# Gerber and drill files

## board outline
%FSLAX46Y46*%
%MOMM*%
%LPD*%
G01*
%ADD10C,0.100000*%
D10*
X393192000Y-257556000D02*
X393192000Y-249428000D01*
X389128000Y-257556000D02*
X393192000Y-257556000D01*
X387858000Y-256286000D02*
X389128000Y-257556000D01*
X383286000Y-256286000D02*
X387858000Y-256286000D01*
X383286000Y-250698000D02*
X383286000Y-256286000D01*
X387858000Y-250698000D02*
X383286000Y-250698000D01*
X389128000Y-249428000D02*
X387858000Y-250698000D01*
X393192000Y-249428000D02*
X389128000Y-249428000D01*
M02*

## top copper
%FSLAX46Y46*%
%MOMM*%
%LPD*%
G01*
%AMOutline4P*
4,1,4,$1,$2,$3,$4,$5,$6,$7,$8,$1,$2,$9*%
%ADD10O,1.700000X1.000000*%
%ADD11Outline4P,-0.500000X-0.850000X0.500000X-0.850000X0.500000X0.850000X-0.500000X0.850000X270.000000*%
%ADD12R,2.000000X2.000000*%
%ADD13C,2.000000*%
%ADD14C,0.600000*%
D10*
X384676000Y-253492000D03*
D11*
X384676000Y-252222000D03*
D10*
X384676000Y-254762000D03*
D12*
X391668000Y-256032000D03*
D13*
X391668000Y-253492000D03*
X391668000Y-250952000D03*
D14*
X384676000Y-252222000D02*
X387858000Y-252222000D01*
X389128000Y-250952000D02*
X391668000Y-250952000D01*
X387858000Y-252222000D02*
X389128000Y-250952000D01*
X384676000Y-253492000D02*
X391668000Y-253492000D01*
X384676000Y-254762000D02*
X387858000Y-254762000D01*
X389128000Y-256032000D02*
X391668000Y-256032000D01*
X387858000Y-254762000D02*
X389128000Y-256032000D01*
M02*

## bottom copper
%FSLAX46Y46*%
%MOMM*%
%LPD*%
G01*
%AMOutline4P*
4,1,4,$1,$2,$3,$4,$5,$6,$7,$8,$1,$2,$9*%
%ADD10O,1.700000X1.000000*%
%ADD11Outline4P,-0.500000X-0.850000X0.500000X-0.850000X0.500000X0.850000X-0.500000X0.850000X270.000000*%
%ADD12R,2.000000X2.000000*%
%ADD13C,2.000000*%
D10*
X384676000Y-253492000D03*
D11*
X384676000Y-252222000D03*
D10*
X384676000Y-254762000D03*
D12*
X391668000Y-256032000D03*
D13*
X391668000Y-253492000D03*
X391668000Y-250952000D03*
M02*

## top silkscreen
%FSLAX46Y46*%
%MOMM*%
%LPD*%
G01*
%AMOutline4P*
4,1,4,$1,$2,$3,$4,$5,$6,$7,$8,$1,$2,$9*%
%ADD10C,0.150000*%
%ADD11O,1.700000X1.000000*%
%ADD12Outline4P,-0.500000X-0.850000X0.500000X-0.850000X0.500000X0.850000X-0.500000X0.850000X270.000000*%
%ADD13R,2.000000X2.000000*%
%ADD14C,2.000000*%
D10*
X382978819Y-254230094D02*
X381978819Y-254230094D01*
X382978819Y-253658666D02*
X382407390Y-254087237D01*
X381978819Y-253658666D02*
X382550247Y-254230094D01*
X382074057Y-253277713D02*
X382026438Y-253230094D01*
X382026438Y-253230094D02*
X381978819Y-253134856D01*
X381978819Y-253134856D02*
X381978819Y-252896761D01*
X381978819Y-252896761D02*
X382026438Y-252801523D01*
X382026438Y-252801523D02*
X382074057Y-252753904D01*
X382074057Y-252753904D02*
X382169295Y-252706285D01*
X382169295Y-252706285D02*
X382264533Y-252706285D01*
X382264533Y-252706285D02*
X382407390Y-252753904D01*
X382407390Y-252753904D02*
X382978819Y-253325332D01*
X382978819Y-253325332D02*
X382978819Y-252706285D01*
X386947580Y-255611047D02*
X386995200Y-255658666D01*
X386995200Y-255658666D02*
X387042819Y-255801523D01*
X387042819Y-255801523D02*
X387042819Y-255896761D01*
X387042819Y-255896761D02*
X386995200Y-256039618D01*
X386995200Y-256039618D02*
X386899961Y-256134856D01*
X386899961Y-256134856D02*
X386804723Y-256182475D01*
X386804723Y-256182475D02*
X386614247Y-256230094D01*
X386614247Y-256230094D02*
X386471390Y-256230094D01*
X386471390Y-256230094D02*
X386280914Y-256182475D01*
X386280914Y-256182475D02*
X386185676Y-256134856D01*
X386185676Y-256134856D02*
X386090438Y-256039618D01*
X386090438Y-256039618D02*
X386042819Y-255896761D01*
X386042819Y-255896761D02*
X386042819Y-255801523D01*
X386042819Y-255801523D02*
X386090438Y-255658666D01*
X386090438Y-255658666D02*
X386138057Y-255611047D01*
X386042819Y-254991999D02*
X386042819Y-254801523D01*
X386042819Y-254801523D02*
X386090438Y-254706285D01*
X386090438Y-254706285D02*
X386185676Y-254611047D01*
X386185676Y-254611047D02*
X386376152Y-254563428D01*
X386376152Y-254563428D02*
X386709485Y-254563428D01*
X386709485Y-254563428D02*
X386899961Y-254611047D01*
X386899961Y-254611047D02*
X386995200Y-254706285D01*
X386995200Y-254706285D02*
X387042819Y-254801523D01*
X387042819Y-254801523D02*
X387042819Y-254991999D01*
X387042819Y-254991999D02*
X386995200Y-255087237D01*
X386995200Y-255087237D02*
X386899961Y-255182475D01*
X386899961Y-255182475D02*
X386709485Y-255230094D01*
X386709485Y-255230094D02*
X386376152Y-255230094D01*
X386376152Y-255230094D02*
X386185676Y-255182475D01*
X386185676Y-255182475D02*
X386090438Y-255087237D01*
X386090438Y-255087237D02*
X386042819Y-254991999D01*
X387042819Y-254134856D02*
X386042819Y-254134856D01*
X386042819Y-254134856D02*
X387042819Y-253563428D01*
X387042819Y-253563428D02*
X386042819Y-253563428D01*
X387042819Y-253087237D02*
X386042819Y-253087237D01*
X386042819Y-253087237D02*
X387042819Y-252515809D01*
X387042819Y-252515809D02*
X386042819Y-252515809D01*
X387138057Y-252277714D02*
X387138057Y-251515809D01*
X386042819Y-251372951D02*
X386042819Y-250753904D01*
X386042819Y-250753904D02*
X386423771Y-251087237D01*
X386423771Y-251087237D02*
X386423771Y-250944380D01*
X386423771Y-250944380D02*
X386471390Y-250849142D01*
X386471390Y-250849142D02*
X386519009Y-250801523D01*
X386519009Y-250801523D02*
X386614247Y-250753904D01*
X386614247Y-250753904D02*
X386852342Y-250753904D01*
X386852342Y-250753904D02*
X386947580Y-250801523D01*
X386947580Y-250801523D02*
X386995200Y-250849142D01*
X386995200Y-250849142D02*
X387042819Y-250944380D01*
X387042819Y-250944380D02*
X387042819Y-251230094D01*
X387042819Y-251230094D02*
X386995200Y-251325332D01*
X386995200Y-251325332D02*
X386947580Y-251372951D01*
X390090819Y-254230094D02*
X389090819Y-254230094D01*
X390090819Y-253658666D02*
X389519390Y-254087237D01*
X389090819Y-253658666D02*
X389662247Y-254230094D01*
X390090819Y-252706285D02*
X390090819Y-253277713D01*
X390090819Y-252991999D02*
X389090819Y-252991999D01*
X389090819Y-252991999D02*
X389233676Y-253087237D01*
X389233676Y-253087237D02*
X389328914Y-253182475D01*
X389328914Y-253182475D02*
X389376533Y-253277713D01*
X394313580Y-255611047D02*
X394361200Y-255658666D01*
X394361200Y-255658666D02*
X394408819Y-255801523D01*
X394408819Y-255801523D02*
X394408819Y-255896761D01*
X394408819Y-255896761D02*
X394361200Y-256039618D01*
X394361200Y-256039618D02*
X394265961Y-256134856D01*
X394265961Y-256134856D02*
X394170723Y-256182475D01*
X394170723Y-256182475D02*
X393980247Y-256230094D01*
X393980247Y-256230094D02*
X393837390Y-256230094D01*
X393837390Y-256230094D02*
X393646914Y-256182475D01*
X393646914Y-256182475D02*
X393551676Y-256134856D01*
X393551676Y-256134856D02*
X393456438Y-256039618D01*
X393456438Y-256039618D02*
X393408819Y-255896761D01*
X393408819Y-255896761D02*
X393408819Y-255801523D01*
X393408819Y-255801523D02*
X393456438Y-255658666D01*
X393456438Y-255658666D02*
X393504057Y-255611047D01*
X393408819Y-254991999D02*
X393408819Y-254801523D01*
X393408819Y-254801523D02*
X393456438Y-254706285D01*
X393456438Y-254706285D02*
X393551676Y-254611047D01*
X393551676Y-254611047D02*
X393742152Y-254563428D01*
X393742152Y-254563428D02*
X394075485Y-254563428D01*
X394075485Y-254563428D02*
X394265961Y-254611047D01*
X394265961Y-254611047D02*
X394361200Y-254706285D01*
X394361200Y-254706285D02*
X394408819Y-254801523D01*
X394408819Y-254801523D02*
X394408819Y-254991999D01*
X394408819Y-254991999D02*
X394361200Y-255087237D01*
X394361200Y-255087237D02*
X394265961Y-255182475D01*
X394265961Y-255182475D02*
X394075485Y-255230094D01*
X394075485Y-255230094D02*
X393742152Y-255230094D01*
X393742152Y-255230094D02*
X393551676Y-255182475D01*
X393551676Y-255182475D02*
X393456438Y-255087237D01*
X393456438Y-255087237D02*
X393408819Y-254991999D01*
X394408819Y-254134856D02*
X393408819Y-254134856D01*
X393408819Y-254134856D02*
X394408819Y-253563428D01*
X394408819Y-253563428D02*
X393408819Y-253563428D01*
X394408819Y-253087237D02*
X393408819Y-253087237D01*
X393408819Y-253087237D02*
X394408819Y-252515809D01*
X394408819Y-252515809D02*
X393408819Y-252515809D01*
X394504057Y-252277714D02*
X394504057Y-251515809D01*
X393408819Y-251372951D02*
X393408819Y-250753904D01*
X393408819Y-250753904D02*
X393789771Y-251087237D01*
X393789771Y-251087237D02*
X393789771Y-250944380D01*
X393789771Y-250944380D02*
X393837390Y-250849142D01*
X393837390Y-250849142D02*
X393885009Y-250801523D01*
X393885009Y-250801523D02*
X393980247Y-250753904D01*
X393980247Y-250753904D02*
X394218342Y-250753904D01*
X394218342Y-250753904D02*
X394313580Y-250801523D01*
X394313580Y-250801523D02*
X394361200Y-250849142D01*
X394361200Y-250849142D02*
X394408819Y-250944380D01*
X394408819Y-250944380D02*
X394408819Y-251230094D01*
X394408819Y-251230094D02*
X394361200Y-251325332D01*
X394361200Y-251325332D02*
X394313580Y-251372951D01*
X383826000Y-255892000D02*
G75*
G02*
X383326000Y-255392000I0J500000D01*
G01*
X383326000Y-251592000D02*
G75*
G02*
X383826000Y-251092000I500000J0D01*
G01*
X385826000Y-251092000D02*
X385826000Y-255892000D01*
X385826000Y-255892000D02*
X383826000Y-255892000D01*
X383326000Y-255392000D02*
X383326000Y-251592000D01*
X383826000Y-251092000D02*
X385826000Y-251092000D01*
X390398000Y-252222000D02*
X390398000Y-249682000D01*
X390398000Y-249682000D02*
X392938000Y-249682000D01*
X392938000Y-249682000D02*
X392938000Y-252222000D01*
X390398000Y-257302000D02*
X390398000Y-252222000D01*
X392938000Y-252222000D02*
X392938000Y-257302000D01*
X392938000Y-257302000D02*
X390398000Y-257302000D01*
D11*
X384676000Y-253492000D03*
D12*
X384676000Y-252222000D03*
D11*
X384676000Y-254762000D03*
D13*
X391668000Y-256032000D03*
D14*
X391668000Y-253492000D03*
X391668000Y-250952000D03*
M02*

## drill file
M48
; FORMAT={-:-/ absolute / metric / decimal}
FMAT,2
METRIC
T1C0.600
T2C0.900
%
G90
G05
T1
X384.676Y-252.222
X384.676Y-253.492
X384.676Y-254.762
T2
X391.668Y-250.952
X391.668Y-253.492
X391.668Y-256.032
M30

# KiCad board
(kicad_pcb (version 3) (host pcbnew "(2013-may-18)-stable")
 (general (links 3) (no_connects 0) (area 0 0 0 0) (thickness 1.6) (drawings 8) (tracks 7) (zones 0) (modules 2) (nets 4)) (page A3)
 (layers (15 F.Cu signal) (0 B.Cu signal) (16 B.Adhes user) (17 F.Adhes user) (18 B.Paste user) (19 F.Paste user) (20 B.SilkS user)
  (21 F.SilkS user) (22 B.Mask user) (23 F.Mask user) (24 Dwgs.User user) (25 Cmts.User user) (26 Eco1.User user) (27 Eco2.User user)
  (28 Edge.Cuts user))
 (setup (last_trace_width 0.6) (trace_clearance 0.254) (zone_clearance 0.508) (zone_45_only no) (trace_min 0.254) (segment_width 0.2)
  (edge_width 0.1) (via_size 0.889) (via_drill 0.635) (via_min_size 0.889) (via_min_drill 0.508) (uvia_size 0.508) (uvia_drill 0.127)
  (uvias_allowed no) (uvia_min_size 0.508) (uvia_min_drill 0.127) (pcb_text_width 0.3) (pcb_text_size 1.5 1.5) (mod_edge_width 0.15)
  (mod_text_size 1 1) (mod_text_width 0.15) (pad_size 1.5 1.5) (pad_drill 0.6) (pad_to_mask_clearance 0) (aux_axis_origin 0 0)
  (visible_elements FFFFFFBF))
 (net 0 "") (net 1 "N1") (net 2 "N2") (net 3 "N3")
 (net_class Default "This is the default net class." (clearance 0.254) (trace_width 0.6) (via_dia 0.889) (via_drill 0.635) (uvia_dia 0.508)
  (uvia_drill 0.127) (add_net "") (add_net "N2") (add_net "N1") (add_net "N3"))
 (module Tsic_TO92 (layer F.Cu) (at 386.588 253.492 270)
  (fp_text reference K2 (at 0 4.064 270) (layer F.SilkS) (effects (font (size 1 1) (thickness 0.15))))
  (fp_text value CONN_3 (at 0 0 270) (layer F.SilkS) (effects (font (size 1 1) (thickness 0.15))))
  (fp_arc (start 1.9 2.762) (end 2.4 2.762) (angle 90) (layer F.SilkS) (width 0.15))
  (fp_arc (start -1.9 2.762) (end -1.9 3.262) (angle 90) (layer F.SilkS) (width 0.15))
  (fp_line (start -2.4 0.762) (end 2.4 0.762) (layer F.SilkS) (width 0.15))
  (fp_line (start 2.4 0.762) (end 2.4 2.762) (layer F.SilkS) (width 0.15))
  (fp_line (start 1.9 3.262) (end -1.9 3.262) (layer F.SilkS) (width 0.15))
  (fp_line (start -2.4 2.762) (end -2.4 0.762) (layer F.SilkS) (width 0.15))
  (pad 2 thru_hole oval (at 0 1.912 270) (size 1 1.7) (drill 0.6) (layers *.Cu *.Mask F.SilkS) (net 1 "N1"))
  (pad 1 thru_hole trapezoid (at -1.27 1.912 270) (size 1 1.7) (drill 0.6) (layers *.Cu *.Mask F.SilkS) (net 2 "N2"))
  (pad 3 thru_hole oval (at 1.27 1.912 270) (size 1 1.7) (drill 0.6) (layers *.Cu *.Mask F.SilkS) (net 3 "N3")))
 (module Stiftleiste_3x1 (layer F.Cu) (at 391.668 253.492 90)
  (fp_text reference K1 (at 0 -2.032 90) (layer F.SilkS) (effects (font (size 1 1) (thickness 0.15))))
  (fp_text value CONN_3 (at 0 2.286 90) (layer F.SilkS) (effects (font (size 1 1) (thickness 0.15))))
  (fp_line (start 1.27 -1.27) (end 3.81 -1.27) (layer F.SilkS) (width 0.15))
  (fp_line (start 3.81 -1.27) (end 3.81 1.27) (layer F.SilkS) (width 0.15))
  (fp_line (start 3.81 1.27) (end 1.27 1.27) (layer F.SilkS) (width 0.15))
  (fp_line (start -3.81 -1.27) (end 1.27 -1.27) (layer F.SilkS) (width 0.15))
  (fp_line (start 1.27 1.27) (end -3.81 1.27) (layer F.SilkS) (width 0.15))
  (fp_line (start -3.81 1.27) (end -3.81 -1.27) (layer F.SilkS) (width 0.15))
  (pad 1 thru_hole rect (at -2.54 0 90) (size 2 2) (drill 0.9) (layers *.Cu *.Mask F.SilkS) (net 3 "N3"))
  (pad 2 thru_hole circle (at 0 0 90) (size 2 2) (drill 0.9) (layers *.Cu *.Mask F.SilkS) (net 1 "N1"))
  (pad 3 thru_hole circle (at 2.54 0 90) (size 2 2) (drill 0.9) (layers *.Cu *.Mask F.SilkS) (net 2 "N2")))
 (gr_line (start 393.192 257.556) (end 393.192 249.428) (angle 90) (layer Edge.Cuts) (width 0.1))
 (gr_line (start 389.128 257.556) (end 393.192 257.556) (angle 90) (layer Edge.Cuts) (width 0.1))
 (gr_line (start 387.858 256.286) (end 389.128 257.556) (angle 90) (layer Edge.Cuts) (width 0.1))
 (gr_line (start 383.286 256.286) (end 387.858 256.286) (angle 90) (layer Edge.Cuts) (width 0.1))
 (gr_line (start 383.286 250.698) (end 383.286 256.286) (angle 90) (layer Edge.Cuts) (width 0.1))
 (gr_line (start 387.858 250.698) (end 383.286 250.698) (angle 90) (layer Edge.Cuts) (width 0.1))
 (gr_line (start 389.128 249.428) (end 387.858 250.698) (angle 90) (layer Edge.Cuts) (width 0.1))
 (gr_line (start 393.192 249.428) (end 389.128 249.428) (angle 90) (layer Edge.Cuts) (width 0.1))
 (segment (start 384.676 252.222) (end 387.858 252.222) (width 0.6) (layer F.Cu) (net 2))
 (segment (start 389.128 250.952) (end 391.668 250.952) (width 0.6) (layer F.Cu) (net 2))
 (segment (start 387.858 252.222) (end 389.128 250.952) (width 0.6) (layer F.Cu) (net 2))
 (segment (start 384.676 253.492) (end 391.668 253.492) (width 0.6) (layer F.Cu) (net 1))
 (segment (start 384.676 254.762) (end 387.858 254.762) (width 0.6) (layer F.Cu) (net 3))
 (segment (start 389.128 256.032) (end 391.668 256.032) (width 0.6) (layer F.Cu) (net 3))
 (segment (start 387.858 254.762) (end 389.128 256.032) (width 0.6) (layer F.Cu) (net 3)))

